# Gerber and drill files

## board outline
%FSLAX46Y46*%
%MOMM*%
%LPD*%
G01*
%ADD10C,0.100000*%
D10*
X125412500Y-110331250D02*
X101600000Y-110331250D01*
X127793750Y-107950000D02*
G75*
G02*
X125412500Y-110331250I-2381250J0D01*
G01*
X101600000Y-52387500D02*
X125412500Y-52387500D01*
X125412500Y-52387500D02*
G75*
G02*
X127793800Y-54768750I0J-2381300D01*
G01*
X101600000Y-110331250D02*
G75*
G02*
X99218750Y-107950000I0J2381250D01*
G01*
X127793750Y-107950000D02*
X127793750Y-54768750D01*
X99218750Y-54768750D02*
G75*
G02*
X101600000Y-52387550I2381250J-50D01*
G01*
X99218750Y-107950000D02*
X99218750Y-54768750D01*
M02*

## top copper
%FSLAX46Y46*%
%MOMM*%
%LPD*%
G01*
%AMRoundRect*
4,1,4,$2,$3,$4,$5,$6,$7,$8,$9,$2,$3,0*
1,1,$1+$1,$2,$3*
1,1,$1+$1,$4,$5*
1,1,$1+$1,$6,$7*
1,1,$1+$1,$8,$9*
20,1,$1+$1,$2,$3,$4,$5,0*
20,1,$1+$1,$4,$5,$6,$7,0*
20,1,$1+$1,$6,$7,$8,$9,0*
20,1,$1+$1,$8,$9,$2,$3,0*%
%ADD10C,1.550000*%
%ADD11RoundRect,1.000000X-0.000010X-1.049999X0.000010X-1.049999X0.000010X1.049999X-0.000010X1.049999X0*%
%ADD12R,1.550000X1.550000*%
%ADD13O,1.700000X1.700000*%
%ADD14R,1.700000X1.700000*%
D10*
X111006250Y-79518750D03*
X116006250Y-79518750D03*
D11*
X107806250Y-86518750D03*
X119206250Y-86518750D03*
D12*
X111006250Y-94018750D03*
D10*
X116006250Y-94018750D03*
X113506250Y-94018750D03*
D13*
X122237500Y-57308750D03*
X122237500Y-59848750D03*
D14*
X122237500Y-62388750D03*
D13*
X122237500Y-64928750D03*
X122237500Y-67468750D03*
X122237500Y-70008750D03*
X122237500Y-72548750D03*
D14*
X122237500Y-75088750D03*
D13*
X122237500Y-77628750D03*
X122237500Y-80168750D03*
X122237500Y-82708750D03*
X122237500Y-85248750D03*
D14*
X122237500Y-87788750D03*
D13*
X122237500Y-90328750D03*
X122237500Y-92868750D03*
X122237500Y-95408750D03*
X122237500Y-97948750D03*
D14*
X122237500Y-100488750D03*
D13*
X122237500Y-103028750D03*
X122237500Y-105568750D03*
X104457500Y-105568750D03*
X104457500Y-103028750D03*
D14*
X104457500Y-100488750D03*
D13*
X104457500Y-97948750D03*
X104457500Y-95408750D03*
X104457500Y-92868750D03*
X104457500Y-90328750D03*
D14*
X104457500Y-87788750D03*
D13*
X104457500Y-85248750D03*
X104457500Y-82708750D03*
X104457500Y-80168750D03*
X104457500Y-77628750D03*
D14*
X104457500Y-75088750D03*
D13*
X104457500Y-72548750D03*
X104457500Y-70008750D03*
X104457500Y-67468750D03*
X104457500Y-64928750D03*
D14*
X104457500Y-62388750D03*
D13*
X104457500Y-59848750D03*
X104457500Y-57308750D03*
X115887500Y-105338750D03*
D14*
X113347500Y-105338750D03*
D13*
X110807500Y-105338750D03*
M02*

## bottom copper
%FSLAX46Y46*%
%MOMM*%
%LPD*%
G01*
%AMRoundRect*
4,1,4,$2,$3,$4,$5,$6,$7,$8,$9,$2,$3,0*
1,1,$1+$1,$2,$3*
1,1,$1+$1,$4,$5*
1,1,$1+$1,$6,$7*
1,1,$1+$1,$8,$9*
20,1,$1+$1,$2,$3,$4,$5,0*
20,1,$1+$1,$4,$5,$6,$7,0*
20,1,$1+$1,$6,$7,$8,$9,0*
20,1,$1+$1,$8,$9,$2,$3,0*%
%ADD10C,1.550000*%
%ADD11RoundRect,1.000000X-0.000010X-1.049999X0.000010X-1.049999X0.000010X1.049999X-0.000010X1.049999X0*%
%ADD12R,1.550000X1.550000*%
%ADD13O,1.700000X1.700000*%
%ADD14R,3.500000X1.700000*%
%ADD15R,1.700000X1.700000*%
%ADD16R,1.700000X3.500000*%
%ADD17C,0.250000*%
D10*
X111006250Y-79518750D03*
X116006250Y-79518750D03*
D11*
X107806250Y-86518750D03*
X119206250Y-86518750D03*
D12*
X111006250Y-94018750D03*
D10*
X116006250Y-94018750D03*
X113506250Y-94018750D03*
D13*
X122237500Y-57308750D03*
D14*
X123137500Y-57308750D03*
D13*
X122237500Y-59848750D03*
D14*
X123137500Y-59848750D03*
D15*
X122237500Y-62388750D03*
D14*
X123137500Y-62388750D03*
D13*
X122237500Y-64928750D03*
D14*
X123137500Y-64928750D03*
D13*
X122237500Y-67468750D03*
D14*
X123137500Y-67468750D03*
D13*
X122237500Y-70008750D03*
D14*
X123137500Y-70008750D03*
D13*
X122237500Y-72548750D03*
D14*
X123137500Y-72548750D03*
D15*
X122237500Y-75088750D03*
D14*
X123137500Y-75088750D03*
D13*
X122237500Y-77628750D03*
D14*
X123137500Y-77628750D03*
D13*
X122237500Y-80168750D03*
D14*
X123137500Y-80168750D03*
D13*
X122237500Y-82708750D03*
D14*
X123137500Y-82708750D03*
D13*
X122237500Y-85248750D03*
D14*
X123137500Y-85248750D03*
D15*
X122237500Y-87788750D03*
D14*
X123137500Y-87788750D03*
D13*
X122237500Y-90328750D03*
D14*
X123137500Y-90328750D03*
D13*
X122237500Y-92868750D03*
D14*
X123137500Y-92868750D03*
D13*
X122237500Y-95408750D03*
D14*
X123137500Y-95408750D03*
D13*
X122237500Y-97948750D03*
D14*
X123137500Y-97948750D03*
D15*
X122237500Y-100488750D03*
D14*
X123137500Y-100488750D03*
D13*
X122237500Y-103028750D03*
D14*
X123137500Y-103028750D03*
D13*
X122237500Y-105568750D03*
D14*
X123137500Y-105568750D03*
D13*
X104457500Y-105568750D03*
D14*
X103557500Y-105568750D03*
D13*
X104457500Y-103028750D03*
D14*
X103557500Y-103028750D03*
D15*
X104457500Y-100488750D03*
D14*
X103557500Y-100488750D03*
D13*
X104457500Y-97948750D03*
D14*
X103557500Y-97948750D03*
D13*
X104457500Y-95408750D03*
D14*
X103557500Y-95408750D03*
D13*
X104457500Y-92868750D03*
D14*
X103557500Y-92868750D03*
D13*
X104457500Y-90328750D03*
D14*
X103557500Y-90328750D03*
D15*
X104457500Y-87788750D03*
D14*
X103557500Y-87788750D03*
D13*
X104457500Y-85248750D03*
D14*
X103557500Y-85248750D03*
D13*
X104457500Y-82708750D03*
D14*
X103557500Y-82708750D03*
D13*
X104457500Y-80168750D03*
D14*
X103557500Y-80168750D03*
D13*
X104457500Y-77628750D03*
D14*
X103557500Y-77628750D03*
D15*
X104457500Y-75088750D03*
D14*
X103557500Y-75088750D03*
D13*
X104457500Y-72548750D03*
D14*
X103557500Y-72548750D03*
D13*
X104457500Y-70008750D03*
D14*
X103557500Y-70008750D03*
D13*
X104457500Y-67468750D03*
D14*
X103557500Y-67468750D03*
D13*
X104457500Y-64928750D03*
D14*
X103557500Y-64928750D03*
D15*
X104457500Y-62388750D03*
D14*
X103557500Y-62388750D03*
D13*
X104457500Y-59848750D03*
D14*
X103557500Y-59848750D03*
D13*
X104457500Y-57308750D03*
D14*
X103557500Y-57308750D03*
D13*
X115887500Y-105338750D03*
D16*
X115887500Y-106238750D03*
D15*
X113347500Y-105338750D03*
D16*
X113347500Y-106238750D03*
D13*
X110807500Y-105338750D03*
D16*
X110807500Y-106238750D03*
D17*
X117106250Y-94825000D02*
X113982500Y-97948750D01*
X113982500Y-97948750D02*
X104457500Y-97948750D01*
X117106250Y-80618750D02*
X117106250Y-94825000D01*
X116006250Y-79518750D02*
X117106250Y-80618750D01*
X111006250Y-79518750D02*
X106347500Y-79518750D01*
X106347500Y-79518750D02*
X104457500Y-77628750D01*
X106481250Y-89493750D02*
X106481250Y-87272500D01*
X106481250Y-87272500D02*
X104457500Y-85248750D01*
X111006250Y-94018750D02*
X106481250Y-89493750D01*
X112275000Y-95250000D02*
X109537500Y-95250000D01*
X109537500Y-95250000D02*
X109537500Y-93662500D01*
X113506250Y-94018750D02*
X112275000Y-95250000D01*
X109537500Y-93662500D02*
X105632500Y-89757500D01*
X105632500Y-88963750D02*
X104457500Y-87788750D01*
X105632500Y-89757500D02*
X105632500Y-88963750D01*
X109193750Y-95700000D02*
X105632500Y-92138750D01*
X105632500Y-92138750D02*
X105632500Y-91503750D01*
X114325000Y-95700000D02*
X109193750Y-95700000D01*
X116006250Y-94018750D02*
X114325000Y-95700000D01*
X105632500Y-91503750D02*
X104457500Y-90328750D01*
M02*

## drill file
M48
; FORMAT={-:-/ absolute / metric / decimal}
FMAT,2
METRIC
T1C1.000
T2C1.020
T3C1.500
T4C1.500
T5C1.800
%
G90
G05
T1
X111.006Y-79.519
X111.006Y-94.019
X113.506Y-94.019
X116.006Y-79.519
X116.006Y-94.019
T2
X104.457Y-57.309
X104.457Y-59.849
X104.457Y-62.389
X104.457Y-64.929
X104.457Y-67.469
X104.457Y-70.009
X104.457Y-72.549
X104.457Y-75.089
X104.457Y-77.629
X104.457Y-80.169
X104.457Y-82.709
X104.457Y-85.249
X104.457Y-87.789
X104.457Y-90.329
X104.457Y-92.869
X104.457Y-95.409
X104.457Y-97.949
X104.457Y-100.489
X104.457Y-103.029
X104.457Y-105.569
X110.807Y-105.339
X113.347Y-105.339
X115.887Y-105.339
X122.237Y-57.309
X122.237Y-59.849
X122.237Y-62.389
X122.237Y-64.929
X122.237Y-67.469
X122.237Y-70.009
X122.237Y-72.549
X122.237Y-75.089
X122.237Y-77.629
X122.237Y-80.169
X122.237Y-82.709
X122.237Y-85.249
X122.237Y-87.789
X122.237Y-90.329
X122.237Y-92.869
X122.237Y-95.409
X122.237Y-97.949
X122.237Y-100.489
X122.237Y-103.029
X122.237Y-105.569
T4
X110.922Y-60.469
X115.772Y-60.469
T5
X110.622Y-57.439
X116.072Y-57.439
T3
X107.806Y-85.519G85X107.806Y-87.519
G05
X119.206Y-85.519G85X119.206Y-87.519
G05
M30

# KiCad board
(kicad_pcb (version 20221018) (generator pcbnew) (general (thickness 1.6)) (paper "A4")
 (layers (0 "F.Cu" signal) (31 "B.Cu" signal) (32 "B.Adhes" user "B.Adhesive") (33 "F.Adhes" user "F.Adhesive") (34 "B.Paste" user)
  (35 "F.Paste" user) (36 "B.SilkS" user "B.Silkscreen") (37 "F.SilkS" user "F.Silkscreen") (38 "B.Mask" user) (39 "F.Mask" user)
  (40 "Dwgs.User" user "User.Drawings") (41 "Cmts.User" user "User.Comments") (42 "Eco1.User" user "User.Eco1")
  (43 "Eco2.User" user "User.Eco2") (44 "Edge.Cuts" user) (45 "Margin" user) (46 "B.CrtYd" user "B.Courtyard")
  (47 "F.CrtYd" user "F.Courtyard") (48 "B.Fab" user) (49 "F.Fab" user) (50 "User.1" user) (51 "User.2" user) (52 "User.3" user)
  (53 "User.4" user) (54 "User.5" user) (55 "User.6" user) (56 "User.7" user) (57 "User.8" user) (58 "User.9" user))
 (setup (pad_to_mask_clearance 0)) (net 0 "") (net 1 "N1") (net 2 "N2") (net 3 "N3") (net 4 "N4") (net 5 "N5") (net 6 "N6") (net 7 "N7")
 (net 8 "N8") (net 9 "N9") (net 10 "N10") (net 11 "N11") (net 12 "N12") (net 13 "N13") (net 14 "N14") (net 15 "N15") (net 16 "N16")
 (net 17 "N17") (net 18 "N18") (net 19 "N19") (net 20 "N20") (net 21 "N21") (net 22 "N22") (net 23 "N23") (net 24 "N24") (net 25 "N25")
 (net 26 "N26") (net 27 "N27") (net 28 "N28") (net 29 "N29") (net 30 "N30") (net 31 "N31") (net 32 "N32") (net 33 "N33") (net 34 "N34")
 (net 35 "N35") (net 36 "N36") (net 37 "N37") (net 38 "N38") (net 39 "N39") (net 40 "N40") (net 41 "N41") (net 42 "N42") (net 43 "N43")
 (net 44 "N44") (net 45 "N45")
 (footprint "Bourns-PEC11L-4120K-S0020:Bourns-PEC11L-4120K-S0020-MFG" (layer "F.Cu") (at 113.50625 86.51875)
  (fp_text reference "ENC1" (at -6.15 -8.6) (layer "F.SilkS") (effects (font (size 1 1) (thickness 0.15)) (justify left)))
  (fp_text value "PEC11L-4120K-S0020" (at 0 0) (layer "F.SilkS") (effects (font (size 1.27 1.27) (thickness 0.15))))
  (pad "1" thru_hole circle (at -2.5 -7) (size 1.55 1.55) (drill 1) (layers "*.Cu") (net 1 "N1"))
  (pad "2" thru_hole circle (at 2.5 -7) (size 1.55 1.55) (drill 1) (layers "*.Cu") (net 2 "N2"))
  (pad "3" thru_hole roundrect (at -5.7 0) (size 2 4.099999) (drill oval 1.5 3.5) (layers "*.Cu") (roundrect_rratio 0.5) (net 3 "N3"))
  (pad "4" thru_hole roundrect (at 5.7 0) (size 2 4.099999) (drill oval 1.5 3.5) (layers "*.Cu") (roundrect_rratio 0.5) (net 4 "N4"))
  (pad "A" thru_hole rect (at -2.5 7.5) (size 1.55 1.55) (drill 1) (layers "*.Cu") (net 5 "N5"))
  (pad "B" thru_hole circle (at 2.5 7.5) (size 1.55 1.55) (drill 1) (layers "*.Cu") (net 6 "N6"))
  (pad "C" thru_hole circle (at 0 7.5) (size 1.55 1.55) (drill 1) (layers "*.Cu") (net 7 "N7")))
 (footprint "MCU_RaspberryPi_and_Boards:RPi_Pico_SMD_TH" (layer "B.Cu") (at 113.3475 81.43875 180)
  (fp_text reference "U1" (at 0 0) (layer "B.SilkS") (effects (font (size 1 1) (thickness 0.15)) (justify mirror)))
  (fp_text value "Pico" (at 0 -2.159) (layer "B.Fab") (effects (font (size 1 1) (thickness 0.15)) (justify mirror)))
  (pad "" np_thru_hole oval (at -2.725 24 180) (size 1.8 1.8) (drill 1.8) (layers "*.Cu" "*.Mask"))
  (pad "" np_thru_hole oval (at -2.425 20.97 180) (size 1.5 1.5) (drill 1.5) (layers "*.Cu" "*.Mask"))
  (pad "" np_thru_hole oval (at 2.425 20.97 180) (size 1.5 1.5) (drill 1.5) (layers "*.Cu" "*.Mask"))
  (pad "" np_thru_hole oval (at 2.725 24 180) (size 1.8 1.8) (drill 1.8) (layers "*.Cu" "*.Mask"))
  (pad "1" thru_hole oval (at -8.89 24.13 180) (size 1.7 1.7) (drill 1.02) (layers "*.Cu" "*.Mask") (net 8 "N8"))
  (pad "1" smd rect (at -8.89 24.13 180) (size 3.5 1.7) (drill (offset -0.9 0)) (layers "B.Cu" "B.Mask") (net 8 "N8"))
  (pad "2" thru_hole oval (at -8.89 21.59 180) (size 1.7 1.7) (drill 1.02) (layers "*.Cu" "*.Mask") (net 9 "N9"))
  (pad "2" smd rect (at -8.89 21.59 180) (size 3.5 1.7) (drill (offset -0.9 0)) (layers "B.Cu" "B.Mask") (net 9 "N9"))
  (pad "3" thru_hole rect (at -8.89 19.05 180) (size 1.7 1.7) (drill 1.02) (layers "*.Cu" "*.Mask") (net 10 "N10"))
  (pad "3" smd rect (at -8.89 19.05 180) (size 3.5 1.7) (drill (offset -0.9 0)) (layers "B.Cu" "B.Mask") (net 10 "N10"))
  (pad "4" thru_hole oval (at -8.89 16.51 180) (size 1.7 1.7) (drill 1.02) (layers "*.Cu" "*.Mask") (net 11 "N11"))
  (pad "4" smd rect (at -8.89 16.51 180) (size 3.5 1.7) (drill (offset -0.9 0)) (layers "B.Cu" "B.Mask") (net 11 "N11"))
  (pad "5" thru_hole oval (at -8.89 13.97 180) (size 1.7 1.7) (drill 1.02) (layers "*.Cu" "*.Mask") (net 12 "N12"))
  (pad "5" smd rect (at -8.89 13.97 180) (size 3.5 1.7) (drill (offset -0.9 0)) (layers "B.Cu" "B.Mask") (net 12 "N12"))
  (pad "6" thru_hole oval (at -8.89 11.43 180) (size 1.7 1.7) (drill 1.02) (layers "*.Cu" "*.Mask") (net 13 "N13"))
  (pad "6" smd rect (at -8.89 11.43 180) (size 3.5 1.7) (drill (offset -0.9 0)) (layers "B.Cu" "B.Mask") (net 13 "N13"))
  (pad "7" thru_hole oval (at -8.89 8.89 180) (size 1.7 1.7) (drill 1.02) (layers "*.Cu" "*.Mask") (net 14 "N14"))
  (pad "7" smd rect (at -8.89 8.89 180) (size 3.5 1.7) (drill (offset -0.9 0)) (layers "B.Cu" "B.Mask") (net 14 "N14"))
  (pad "8" thru_hole rect (at -8.89 6.35 180) (size 1.7 1.7) (drill 1.02) (layers "*.Cu" "*.Mask") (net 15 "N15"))
  (pad "8" smd rect (at -8.89 6.35 180) (size 3.5 1.7) (drill (offset -0.9 0)) (layers "B.Cu" "B.Mask") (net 15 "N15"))
  (pad "9" thru_hole oval (at -8.89 3.81 180) (size 1.7 1.7) (drill 1.02) (layers "*.Cu" "*.Mask") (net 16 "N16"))
  (pad "9" smd rect (at -8.89 3.81 180) (size 3.5 1.7) (drill (offset -0.9 0)) (layers "B.Cu" "B.Mask") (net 16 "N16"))
  (pad "10" thru_hole oval (at -8.89 1.27 180) (size 1.7 1.7) (drill 1.02) (layers "*.Cu" "*.Mask") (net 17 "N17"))
  (pad "10" smd rect (at -8.89 1.27 180) (size 3.5 1.7) (drill (offset -0.9 0)) (layers "B.Cu" "B.Mask") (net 17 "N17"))
  (pad "11" thru_hole oval (at -8.89 -1.27 180) (size 1.7 1.7) (drill 1.02) (layers "*.Cu" "*.Mask") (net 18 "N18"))
  (pad "11" smd rect (at -8.89 -1.27 180) (size 3.5 1.7) (drill (offset -0.9 0)) (layers "B.Cu" "B.Mask") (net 18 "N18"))
  (pad "12" thru_hole oval (at -8.89 -3.81 180) (size 1.7 1.7) (drill 1.02) (layers "*.Cu" "*.Mask") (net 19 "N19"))
  (pad "12" smd rect (at -8.89 -3.81 180) (size 3.5 1.7) (drill (offset -0.9 0)) (layers "B.Cu" "B.Mask") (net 19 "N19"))
  (pad "13" thru_hole rect (at -8.89 -6.35 180) (size 1.7 1.7) (drill 1.02) (layers "*.Cu" "*.Mask") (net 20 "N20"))
  (pad "13" smd rect (at -8.89 -6.35 180) (size 3.5 1.7) (drill (offset -0.9 0)) (layers "B.Cu" "B.Mask") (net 20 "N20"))
  (pad "14" thru_hole oval (at -8.89 -8.89 180) (size 1.7 1.7) (drill 1.02) (layers "*.Cu" "*.Mask") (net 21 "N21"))
  (pad "14" smd rect (at -8.89 -8.89 180) (size 3.5 1.7) (drill (offset -0.9 0)) (layers "B.Cu" "B.Mask") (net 21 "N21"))
  (pad "15" thru_hole oval (at -8.89 -11.43 180) (size 1.7 1.7) (drill 1.02) (layers "*.Cu" "*.Mask") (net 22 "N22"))
  (pad "15" smd rect (at -8.89 -11.43 180) (size 3.5 1.7) (drill (offset -0.9 0)) (layers "B.Cu" "B.Mask") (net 22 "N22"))
  (pad "16" thru_hole oval (at -8.89 -13.97 180) (size 1.7 1.7) (drill 1.02) (layers "*.Cu" "*.Mask") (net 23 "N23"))
  (pad "16" smd rect (at -8.89 -13.97 180) (size 3.5 1.7) (drill (offset -0.9 0)) (layers "B.Cu" "B.Mask") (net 23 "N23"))
  (pad "17" thru_hole oval (at -8.89 -16.51 180) (size 1.7 1.7) (drill 1.02) (layers "*.Cu" "*.Mask") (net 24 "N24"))
  (pad "17" smd rect (at -8.89 -16.51 180) (size 3.5 1.7) (drill (offset -0.9 0)) (layers "B.Cu" "B.Mask") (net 24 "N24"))
  (pad "18" thru_hole rect (at -8.89 -19.05 180) (size 1.7 1.7) (drill 1.02) (layers "*.Cu" "*.Mask") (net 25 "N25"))
  (pad "18" smd rect (at -8.89 -19.05 180) (size 3.5 1.7) (drill (offset -0.9 0)) (layers "B.Cu" "B.Mask") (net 25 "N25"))
  (pad "19" thru_hole oval (at -8.89 -21.59 180) (size 1.7 1.7) (drill 1.02) (layers "*.Cu" "*.Mask") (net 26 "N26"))
  (pad "19" smd rect (at -8.89 -21.59 180) (size 3.5 1.7) (drill (offset -0.9 0)) (layers "B.Cu" "B.Mask") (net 26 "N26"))
  (pad "20" thru_hole oval (at -8.89 -24.13 180) (size 1.7 1.7) (drill 1.02) (layers "*.Cu" "*.Mask") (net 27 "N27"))
  (pad "20" smd rect (at -8.89 -24.13 180) (size 3.5 1.7) (drill (offset -0.9 0)) (layers "B.Cu" "B.Mask") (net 27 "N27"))
  (pad "21" thru_hole oval (at 8.89 -24.13 180) (size 1.7 1.7) (drill 1.02) (layers "*.Cu" "*.Mask") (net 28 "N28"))
  (pad "21" smd rect (at 8.89 -24.13 180) (size 3.5 1.7) (drill (offset 0.9 0)) (layers "B.Cu" "B.Mask") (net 28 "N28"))
  (pad "22" thru_hole oval (at 8.89 -21.59 180) (size 1.7 1.7) (drill 1.02) (layers "*.Cu" "*.Mask") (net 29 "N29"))
  (pad "22" smd rect (at 8.89 -21.59 180) (size 3.5 1.7) (drill (offset 0.9 0)) (layers "B.Cu" "B.Mask") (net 29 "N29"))
  (pad "23" thru_hole rect (at 8.89 -19.05 180) (size 1.7 1.7) (drill 1.02) (layers "*.Cu" "*.Mask") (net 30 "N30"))
  (pad "23" smd rect (at 8.89 -19.05 180) (size 3.5 1.7) (drill (offset 0.9 0)) (layers "B.Cu" "B.Mask") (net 30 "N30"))
  (pad "24" thru_hole oval (at 8.89 -16.51 180) (size 1.7 1.7) (drill 1.02) (layers "*.Cu" "*.Mask") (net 2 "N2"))
  (pad "24" smd rect (at 8.89 -16.51 180) (size 3.5 1.7) (drill (offset 0.9 0)) (layers "B.Cu" "B.Mask") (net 2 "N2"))
  (pad "25" thru_hole oval (at 8.89 -13.97 180) (size 1.7 1.7) (drill 1.02) (layers "*.Cu" "*.Mask") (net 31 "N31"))
  (pad "25" smd rect (at 8.89 -13.97 180) (size 3.5 1.7) (drill (offset 0.9 0)) (layers "B.Cu" "B.Mask") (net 31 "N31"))
  (pad "26" thru_hole oval (at 8.89 -11.43 180) (size 1.7 1.7) (drill 1.02) (layers "*.Cu" "*.Mask") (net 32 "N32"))
  (pad "26" smd rect (at 8.89 -11.43 180) (size 3.5 1.7) (drill (offset 0.9 0)) (layers "B.Cu" "B.Mask") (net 32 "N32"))
  (pad "27" thru_hole oval (at 8.89 -8.89 180) (size 1.7 1.7) (drill 1.02) (layers "*.Cu" "*.Mask") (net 6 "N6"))
  (pad "27" smd rect (at 8.89 -8.89 180) (size 3.5 1.7) (drill (offset 0.9 0)) (layers "B.Cu" "B.Mask") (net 6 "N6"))
  (pad "28" thru_hole rect (at 8.89 -6.35 180) (size 1.7 1.7) (drill 1.02) (layers "*.Cu" "*.Mask") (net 7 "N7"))
  (pad "28" smd rect (at 8.89 -6.35 180) (size 3.5 1.7) (drill (offset 0.9 0)) (layers "B.Cu" "B.Mask") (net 7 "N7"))
  (pad "29" thru_hole oval (at 8.89 -3.81 180) (size 1.7 1.7) (drill 1.02) (layers "*.Cu" "*.Mask") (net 5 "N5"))
  (pad "29" smd rect (at 8.89 -3.81 180) (size 3.5 1.7) (drill (offset 0.9 0)) (layers "B.Cu" "B.Mask") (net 5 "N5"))
  (pad "30" thru_hole oval (at 8.89 -1.27 180) (size 1.7 1.7) (drill 1.02) (layers "*.Cu" "*.Mask") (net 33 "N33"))
  (pad "30" smd rect (at 8.89 -1.27 180) (size 3.5 1.7) (drill (offset 0.9 0)) (layers "B.Cu" "B.Mask") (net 33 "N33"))
  (pad "31" thru_hole oval (at 8.89 1.27 180) (size 1.7 1.7) (drill 1.02) (layers "*.Cu" "*.Mask") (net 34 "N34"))
  (pad "31" smd rect (at 8.89 1.27 180) (size 3.5 1.7) (drill (offset 0.9 0)) (layers "B.Cu" "B.Mask") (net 34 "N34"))
  (pad "32" thru_hole oval (at 8.89 3.81 180) (size 1.7 1.7) (drill 1.02) (layers "*.Cu" "*.Mask") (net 1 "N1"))
  (pad "32" smd rect (at 8.89 3.81 180) (size 3.5 1.7) (drill (offset 0.9 0)) (layers "B.Cu" "B.Mask") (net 1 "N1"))
  (pad "33" thru_hole rect (at 8.89 6.35 180) (size 1.7 1.7) (drill 1.02) (layers "*.Cu" "*.Mask") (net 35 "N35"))
  (pad "33" smd rect (at 8.89 6.35 180) (size 3.5 1.7) (drill (offset 0.9 0)) (layers "B.Cu" "B.Mask") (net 35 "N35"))
  (pad "34" thru_hole oval (at 8.89 8.89 180) (size 1.7 1.7) (drill 1.02) (layers "*.Cu" "*.Mask") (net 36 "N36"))
  (pad "34" smd rect (at 8.89 8.89 180) (size 3.5 1.7) (drill (offset 0.9 0)) (layers "B.Cu" "B.Mask") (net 36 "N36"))
  (pad "35" thru_hole oval (at 8.89 11.43 180) (size 1.7 1.7) (drill 1.02) (layers "*.Cu" "*.Mask") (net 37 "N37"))
  (pad "35" smd rect (at 8.89 11.43 180) (size 3.5 1.7) (drill (offset 0.9 0)) (layers "B.Cu" "B.Mask") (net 37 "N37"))
  (pad "36" thru_hole oval (at 8.89 13.97 180) (size 1.7 1.7) (drill 1.02) (layers "*.Cu" "*.Mask") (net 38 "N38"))
  (pad "36" smd rect (at 8.89 13.97 180) (size 3.5 1.7) (drill (offset 0.9 0)) (layers "B.Cu" "B.Mask") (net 38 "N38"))
  (pad "37" thru_hole oval (at 8.89 16.51 180) (size 1.7 1.7) (drill 1.02) (layers "*.Cu" "*.Mask") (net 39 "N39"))
  (pad "37" smd rect (at 8.89 16.51 180) (size 3.5 1.7) (drill (offset 0.9 0)) (layers "B.Cu" "B.Mask") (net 39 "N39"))
  (pad "38" thru_hole rect (at 8.89 19.05 180) (size 1.7 1.7) (drill 1.02) (layers "*.Cu" "*.Mask") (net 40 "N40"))
  (pad "38" smd rect (at 8.89 19.05 180) (size 3.5 1.7) (drill (offset 0.9 0)) (layers "B.Cu" "B.Mask") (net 40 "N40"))
  (pad "39" thru_hole oval (at 8.89 21.59 180) (size 1.7 1.7) (drill 1.02) (layers "*.Cu" "*.Mask") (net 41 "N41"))
  (pad "39" smd rect (at 8.89 21.59 180) (size 3.5 1.7) (drill (offset 0.9 0)) (layers "B.Cu" "B.Mask") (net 41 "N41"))
  (pad "40" thru_hole oval (at 8.89 24.13 180) (size 1.7 1.7) (drill 1.02) (layers "*.Cu" "*.Mask") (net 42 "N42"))
  (pad "40" smd rect (at 8.89 24.13 180) (size 3.5 1.7) (drill (offset 0.9 0)) (layers "B.Cu" "B.Mask") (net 42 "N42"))
  (pad "41" thru_hole oval (at -2.54 -23.9 180) (size 1.7 1.7) (drill 1.02) (layers "*.Cu" "*.Mask") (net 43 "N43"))
  (pad "41" smd rect (at -2.54 -23.9 90) (size 3.5 1.7) (drill (offset -0.9 0)) (layers "B.Cu" "B.Mask") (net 43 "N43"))
  (pad "42" thru_hole rect (at 0 -23.9 180) (size 1.7 1.7) (drill 1.02) (layers "*.Cu" "*.Mask") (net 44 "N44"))
  (pad "42" smd rect (at 0 -23.9 90) (size 3.5 1.7) (drill (offset -0.9 0)) (layers "B.Cu" "B.Mask") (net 44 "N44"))
  (pad "43" thru_hole oval (at 2.54 -23.9 180) (size 1.7 1.7) (drill 1.02) (layers "*.Cu" "*.Mask") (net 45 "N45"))
  (pad "43" smd rect (at 2.54 -23.9 90) (size 3.5 1.7) (drill (offset -0.9 0)) (layers "B.Cu" "B.Mask") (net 45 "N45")))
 (gr_line (start 125.4125 110.33125) (end 101.6 110.33125) (stroke (width 0.1) (type default)) (layer "Edge.Cuts"))
 (gr_arc (start 127.79375 107.95) (mid 127.096298 109.633798) (end 125.4125 110.33125) (stroke (width 0.1) (type default))
  (layer "Edge.Cuts"))
 (gr_line (start 101.6 52.3875) (end 125.4125 52.3875) (stroke (width 0.1) (type default)) (layer "Edge.Cuts"))
 (gr_arc (start 125.4125 52.3875) (mid 127.096298 53.084952) (end 127.79375 54.76875) (stroke (width 0.1) (type default))
  (layer "Edge.Cuts"))
 (gr_arc (start 101.6 110.33125) (mid 99.916202 109.633798) (end 99.21875 107.95) (stroke (width 0.1) (type default)) (layer "Edge.Cuts"))
 (gr_line (start 127.79375 107.95) (end 127.79375 54.76875) (stroke (width 0.1) (type default)) (layer "Edge.Cuts"))
 (gr_arc (start 99.21875 54.76875) (mid 99.916202 53.084952) (end 101.6 52.3875) (stroke (width 0.1) (type default)) (layer "Edge.Cuts"))
 (gr_line (start 99.21875 107.95) (end 99.21875 54.76875) (stroke (width 0.1) (type default)) (layer "Edge.Cuts"))
 (segment (start 117.10625 94.825) (end 113.9825 97.94875) (width 0.25) (layer "B.Cu") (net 2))
 (segment (start 113.9825 97.94875) (end 104.4575 97.94875) (width 0.25) (layer "B.Cu") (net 2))
 (segment (start 117.10625 80.61875) (end 117.10625 94.825) (width 0.25) (layer "B.Cu") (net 2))
 (segment (start 116.00625 79.51875) (end 117.10625 80.61875) (width 0.25) (layer "B.Cu") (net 2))
 (segment (start 111.00625 79.51875) (end 106.3475 79.51875) (width 0.25) (layer "B.Cu") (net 1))
 (segment (start 106.3475 79.51875) (end 104.4575 77.62875) (width 0.25) (layer "B.Cu") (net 1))
 (segment (start 106.48125 89.49375) (end 106.48125 87.2725) (width 0.25) (layer "B.Cu") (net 5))
 (segment (start 106.48125 87.2725) (end 104.4575 85.24875) (width 0.25) (layer "B.Cu") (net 5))
 (segment (start 111.00625 94.01875) (end 106.48125 89.49375) (width 0.25) (layer "B.Cu") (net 5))
 (segment (start 112.275 95.25) (end 109.5375 95.25) (width 0.25) (layer "B.Cu") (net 7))
 (segment (start 109.5375 95.25) (end 109.5375 93.6625) (width 0.25) (layer "B.Cu") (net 7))
 (segment (start 113.50625 94.01875) (end 112.275 95.25) (width 0.25) (layer "B.Cu") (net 7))
 (segment (start 109.5375 93.6625) (end 105.6325 89.7575) (width 0.25) (layer "B.Cu") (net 7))
 (segment (start 105.6325 88.96375) (end 104.4575 87.78875) (width 0.25) (layer "B.Cu") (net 7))
 (segment (start 105.6325 89.7575) (end 105.6325 88.96375) (width 0.25) (layer "B.Cu") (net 7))
 (segment (start 109.19375 95.7) (end 105.6325 92.13875) (width 0.25) (layer "B.Cu") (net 6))
 (segment (start 105.6325 92.13875) (end 105.6325 91.50375) (width 0.25) (layer "B.Cu") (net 6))
 (segment (start 114.325 95.7) (end 109.19375 95.7) (width 0.25) (layer "B.Cu") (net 6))
 (segment (start 116.00625 94.01875) (end 114.325 95.7) (width 0.25) (layer "B.Cu") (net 6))
 (segment (start 105.6325 91.50375) (end 104.4575 90.32875) (width 0.25) (layer "B.Cu") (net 6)))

